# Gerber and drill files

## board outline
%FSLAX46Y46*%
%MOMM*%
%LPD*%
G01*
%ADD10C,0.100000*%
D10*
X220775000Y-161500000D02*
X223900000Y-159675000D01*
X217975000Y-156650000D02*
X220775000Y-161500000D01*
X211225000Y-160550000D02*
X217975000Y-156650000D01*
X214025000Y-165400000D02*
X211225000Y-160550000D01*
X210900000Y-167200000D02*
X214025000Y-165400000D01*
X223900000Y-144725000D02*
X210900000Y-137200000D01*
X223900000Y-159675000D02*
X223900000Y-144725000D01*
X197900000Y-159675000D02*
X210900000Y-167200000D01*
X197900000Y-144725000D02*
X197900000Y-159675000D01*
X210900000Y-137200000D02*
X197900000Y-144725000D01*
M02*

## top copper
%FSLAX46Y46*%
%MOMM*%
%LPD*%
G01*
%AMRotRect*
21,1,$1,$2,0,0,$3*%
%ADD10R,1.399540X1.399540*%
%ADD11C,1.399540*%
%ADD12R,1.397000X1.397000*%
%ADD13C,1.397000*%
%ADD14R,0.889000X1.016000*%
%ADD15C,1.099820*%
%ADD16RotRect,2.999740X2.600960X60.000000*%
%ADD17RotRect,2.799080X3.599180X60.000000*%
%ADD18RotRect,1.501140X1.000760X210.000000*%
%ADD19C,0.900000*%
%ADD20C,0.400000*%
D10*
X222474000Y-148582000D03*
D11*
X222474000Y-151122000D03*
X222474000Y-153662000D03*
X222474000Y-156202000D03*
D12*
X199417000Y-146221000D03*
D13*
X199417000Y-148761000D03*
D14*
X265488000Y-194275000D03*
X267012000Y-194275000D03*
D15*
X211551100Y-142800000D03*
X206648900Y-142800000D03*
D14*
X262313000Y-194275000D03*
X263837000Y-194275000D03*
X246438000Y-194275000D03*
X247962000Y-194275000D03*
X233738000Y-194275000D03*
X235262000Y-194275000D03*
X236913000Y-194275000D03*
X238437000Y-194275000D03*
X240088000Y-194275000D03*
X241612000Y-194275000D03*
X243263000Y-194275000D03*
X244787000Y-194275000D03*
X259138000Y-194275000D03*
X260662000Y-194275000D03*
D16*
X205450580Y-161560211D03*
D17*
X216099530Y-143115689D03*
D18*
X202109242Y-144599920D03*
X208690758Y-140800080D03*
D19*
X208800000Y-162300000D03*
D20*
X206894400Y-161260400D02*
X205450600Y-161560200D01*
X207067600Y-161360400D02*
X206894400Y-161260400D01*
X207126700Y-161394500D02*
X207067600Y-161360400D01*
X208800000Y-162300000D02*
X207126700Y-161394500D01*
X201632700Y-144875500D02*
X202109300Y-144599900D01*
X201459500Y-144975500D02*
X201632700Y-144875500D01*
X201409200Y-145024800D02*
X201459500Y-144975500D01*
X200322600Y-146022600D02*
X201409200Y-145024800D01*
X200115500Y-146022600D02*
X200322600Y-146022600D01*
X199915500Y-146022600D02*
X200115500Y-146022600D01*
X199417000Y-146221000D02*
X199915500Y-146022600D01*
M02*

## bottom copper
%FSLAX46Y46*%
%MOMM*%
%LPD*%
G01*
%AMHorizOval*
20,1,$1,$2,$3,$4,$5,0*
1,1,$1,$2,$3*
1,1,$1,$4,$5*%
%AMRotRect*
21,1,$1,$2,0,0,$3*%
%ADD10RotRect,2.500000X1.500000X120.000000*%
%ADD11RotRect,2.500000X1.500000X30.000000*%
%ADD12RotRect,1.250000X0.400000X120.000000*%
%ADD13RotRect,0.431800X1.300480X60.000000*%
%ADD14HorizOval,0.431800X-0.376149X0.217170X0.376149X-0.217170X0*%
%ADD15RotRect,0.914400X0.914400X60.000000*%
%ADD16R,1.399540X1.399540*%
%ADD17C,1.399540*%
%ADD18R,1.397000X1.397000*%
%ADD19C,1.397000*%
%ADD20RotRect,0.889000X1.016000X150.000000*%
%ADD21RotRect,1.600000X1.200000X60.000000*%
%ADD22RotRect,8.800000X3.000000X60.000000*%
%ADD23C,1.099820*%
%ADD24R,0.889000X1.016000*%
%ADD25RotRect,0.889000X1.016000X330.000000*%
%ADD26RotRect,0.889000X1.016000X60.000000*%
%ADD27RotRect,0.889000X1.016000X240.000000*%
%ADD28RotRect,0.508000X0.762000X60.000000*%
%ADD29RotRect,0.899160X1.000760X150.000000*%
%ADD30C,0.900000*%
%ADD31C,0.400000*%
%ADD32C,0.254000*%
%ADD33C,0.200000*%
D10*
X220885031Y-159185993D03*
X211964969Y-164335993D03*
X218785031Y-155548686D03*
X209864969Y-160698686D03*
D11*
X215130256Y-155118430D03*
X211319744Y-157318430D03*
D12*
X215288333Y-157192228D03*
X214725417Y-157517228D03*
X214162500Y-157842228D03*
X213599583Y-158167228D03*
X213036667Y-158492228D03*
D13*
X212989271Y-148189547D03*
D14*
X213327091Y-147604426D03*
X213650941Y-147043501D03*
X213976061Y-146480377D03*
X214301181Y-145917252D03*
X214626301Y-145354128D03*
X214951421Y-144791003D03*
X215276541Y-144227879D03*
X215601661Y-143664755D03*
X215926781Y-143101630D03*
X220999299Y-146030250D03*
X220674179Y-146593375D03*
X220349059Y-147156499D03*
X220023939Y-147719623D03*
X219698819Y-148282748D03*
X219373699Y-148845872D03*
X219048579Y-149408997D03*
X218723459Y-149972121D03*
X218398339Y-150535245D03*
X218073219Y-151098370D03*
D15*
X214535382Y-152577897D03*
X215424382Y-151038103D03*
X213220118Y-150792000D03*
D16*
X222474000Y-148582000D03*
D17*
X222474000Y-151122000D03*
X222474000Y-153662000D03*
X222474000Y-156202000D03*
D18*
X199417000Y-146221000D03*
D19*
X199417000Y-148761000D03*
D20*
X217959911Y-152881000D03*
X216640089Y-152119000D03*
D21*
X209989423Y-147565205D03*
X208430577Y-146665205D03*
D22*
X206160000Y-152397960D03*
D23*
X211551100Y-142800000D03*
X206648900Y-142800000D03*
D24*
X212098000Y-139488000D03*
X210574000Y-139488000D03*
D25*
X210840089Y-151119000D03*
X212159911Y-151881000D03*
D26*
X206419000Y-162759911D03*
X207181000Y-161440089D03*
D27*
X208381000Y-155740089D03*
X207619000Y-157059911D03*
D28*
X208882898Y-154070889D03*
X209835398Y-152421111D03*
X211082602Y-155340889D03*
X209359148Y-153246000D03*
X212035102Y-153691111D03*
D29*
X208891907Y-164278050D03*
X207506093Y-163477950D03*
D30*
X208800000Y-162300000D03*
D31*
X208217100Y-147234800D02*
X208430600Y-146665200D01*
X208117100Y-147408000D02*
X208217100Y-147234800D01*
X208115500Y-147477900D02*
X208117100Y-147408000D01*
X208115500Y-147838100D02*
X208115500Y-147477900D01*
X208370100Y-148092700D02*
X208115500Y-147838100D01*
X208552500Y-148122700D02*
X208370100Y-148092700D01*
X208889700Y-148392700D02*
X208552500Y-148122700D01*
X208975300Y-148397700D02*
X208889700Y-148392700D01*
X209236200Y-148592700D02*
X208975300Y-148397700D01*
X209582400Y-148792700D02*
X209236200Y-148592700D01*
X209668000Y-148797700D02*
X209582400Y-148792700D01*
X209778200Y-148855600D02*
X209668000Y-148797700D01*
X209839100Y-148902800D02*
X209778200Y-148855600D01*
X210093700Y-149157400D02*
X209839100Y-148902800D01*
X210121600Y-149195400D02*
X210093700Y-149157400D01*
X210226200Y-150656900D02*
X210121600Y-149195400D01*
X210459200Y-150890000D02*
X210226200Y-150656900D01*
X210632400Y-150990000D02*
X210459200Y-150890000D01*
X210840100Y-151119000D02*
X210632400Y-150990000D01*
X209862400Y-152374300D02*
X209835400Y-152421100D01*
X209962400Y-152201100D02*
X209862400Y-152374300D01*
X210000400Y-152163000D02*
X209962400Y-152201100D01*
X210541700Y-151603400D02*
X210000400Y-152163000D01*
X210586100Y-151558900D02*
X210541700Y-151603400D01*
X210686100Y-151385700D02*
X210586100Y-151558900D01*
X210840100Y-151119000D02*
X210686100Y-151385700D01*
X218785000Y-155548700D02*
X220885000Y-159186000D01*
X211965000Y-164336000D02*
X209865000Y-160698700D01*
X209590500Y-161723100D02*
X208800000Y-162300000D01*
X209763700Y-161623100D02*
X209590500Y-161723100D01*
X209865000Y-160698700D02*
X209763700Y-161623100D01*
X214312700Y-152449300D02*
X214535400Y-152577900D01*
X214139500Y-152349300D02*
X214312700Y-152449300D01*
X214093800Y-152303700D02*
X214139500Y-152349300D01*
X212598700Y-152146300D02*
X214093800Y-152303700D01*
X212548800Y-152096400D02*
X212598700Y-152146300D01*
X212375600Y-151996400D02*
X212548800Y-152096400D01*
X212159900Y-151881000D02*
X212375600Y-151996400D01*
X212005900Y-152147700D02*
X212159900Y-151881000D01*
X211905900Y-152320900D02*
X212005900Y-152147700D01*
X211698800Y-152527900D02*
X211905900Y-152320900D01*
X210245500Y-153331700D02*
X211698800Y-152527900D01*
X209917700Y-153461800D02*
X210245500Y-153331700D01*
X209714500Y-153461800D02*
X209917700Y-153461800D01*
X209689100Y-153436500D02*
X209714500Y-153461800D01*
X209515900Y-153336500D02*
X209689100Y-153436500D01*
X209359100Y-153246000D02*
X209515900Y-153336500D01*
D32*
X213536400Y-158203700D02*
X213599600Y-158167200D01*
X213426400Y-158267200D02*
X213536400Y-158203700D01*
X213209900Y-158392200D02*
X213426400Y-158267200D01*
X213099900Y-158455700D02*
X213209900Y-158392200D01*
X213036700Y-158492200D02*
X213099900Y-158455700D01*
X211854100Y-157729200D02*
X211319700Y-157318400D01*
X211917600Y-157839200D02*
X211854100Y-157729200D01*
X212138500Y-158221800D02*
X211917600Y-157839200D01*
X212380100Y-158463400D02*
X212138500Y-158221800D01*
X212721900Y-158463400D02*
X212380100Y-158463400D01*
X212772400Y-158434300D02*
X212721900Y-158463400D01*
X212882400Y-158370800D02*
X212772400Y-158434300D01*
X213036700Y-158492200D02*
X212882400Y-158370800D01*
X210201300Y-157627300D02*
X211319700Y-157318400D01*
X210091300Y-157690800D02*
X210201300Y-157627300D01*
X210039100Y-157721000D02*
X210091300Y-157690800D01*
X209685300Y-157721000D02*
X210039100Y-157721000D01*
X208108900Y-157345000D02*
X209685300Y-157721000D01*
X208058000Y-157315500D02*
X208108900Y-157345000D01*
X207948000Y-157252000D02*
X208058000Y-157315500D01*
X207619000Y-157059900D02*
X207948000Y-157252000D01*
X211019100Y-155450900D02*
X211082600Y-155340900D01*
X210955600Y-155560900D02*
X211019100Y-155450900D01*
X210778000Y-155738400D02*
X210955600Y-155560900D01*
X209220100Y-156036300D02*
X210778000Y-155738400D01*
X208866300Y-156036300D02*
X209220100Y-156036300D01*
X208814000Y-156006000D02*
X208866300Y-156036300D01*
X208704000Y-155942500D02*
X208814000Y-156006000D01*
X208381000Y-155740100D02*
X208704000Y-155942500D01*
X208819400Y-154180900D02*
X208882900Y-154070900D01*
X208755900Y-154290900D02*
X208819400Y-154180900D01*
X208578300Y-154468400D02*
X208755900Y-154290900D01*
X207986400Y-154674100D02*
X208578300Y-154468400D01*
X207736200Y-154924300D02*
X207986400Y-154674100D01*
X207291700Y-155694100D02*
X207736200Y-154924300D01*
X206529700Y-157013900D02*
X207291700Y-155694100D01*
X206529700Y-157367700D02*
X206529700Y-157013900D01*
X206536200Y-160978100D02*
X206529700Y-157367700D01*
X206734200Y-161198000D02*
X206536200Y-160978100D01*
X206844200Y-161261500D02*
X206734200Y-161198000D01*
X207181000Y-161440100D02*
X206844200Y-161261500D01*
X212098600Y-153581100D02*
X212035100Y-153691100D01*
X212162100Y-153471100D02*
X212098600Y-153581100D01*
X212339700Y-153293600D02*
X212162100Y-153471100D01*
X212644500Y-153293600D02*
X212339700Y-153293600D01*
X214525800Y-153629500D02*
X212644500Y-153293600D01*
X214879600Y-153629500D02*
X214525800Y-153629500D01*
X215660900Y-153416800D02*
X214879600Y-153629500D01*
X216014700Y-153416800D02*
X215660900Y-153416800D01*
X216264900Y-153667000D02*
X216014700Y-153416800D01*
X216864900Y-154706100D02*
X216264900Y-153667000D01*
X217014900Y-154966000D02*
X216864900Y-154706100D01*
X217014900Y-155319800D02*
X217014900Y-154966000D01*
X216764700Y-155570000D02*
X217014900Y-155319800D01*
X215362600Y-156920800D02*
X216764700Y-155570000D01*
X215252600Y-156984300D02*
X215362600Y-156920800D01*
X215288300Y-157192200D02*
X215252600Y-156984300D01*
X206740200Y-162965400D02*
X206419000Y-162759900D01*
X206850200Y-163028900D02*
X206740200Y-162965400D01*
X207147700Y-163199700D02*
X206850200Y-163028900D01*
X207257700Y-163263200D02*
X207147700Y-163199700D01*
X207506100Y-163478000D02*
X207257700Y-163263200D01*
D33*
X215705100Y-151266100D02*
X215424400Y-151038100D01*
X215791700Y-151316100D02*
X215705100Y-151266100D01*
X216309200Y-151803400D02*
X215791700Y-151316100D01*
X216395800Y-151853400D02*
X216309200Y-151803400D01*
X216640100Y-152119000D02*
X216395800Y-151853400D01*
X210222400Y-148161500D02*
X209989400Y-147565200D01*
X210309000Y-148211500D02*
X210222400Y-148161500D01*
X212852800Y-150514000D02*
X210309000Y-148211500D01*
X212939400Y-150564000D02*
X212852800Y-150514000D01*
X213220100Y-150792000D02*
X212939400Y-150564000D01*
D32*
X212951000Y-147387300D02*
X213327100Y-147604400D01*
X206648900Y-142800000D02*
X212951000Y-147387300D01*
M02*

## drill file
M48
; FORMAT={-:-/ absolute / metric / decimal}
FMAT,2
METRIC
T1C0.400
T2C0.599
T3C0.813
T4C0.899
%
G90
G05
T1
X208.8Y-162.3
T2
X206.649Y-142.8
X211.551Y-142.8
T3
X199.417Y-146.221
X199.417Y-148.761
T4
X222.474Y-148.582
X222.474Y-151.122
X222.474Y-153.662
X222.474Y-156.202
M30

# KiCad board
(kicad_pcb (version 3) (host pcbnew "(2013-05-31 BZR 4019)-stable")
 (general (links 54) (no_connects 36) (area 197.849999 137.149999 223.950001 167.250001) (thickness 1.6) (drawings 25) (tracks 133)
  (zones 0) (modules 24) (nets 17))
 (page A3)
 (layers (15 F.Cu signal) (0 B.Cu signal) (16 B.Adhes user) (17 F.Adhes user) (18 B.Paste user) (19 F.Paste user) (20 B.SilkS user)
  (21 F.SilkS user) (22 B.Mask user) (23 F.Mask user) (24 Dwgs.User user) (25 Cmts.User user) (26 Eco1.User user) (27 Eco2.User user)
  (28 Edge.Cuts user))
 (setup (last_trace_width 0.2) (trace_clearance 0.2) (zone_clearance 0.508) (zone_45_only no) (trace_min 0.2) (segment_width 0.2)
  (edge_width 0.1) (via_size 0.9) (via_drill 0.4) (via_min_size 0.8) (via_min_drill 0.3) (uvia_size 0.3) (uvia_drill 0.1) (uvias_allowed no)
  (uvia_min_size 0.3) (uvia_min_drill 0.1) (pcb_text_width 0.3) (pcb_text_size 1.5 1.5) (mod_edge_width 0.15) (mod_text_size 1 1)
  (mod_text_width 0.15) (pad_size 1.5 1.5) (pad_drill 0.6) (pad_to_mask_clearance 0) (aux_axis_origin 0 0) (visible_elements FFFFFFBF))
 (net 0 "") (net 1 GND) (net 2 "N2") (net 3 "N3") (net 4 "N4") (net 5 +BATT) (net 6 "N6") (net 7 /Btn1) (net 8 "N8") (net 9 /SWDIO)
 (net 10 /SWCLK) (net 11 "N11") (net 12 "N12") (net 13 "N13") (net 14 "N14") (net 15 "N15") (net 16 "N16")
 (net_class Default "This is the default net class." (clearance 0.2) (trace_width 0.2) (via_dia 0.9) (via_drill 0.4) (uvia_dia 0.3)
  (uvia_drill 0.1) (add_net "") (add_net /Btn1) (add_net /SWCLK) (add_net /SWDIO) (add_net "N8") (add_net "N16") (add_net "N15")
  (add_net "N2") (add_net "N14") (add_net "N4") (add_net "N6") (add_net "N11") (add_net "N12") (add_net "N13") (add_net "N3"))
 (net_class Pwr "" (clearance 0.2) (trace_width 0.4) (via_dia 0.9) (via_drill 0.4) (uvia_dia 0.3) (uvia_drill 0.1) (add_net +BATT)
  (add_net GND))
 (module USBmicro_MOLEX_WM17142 (layer B.Cu) (at 214.6 158.6 120)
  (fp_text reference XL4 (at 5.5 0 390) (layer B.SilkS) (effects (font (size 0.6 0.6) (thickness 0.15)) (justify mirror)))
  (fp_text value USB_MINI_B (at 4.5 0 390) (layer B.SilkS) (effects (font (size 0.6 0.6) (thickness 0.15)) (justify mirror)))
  (pad SHLD smd rect (at -3.65 5.15 120) (size 2.5 1.5) (layers B.Cu B.Paste B.Mask) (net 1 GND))
  (pad SHLD smd rect (at -3.65 -5.15 120) (size 2.5 1.5) (layers B.Cu B.Paste B.Mask) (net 1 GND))
  (pad SHLD smd rect (at 0.55 5.15 120) (size 2.5 1.5) (layers B.Cu B.Paste B.Mask) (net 1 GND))
  (pad SHLD smd rect (at 0.55 -5.15 120) (size 2.5 1.5) (layers B.Cu B.Paste B.Mask) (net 1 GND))
  (pad SHLD smd rect (at 2.75 2.2 30) (size 2.5 1.5) (layers B.Cu B.Paste B.Mask) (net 1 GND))
  (pad SHLD smd rect (at 2.75 -2.2 30) (size 2.5 1.5) (layers B.Cu B.Paste B.Mask) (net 1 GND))
  (pad 1 smd rect (at 0.875 1.3 120) (size 1.25 0.4) (layers B.Cu B.Paste B.Mask) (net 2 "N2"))
  (pad 2 smd rect (at 0.875 0.65 120) (size 1.25 0.4) (layers B.Cu B.Paste B.Mask))
  (pad 3 smd rect (at 0.875 0 120) (size 1.25 0.4) (layers B.Cu B.Paste B.Mask))
  (pad 4 smd rect (at 0.875 -0.65 120) (size 1.25 0.4) (layers B.Cu B.Paste B.Mask) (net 1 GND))
  (pad 5 smd rect (at 0.875 -1.3 120) (size 1.25 0.4) (layers B.Cu B.Paste B.Mask) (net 1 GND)))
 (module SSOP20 (layer B.Cu) (at 217 147.1 60)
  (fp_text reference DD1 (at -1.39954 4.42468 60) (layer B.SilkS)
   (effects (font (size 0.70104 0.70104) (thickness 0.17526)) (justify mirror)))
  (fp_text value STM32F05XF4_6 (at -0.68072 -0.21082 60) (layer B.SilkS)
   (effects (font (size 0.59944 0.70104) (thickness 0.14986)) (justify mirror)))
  (pad 1 smd rect (at -2.94894 -2.92862 60) (size 0.4318 1.30048) (layers B.Cu B.Paste B.Mask) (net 1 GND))
  (pad 2 smd oval (at -2.2733 -2.92862 60) (size 0.4318 1.30048) (layers B.Cu B.Paste B.Mask) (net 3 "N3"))
  (pad 3 smd oval (at -1.6256 -2.92862 60) (size 0.4318 1.30048) (layers B.Cu B.Paste B.Mask) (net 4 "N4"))
  (pad 4 smd oval (at -0.97536 -2.92862 60) (size 0.4318 1.30048) (layers B.Cu B.Paste B.Mask))
  (pad 5 smd oval (at -0.32512 -2.92862 60) (size 0.4318 1.30048) (layers B.Cu B.Paste B.Mask) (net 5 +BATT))
  (pad 6 smd oval (at 0.32512 -2.92862 60) (size 0.4318 1.30048) (layers B.Cu B.Paste B.Mask))
  (pad 7 smd oval (at 0.97536 -2.92862 60) (size 0.4318 1.30048) (layers B.Cu B.Paste B.Mask) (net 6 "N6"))
  (pad 8 smd oval (at 1.6256 -2.92862 60) (size 0.4318 1.30048) (layers B.Cu B.Paste B.Mask) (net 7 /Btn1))
  (pad 9 smd oval (at 2.27584 -2.92862 60) (size 0.4318 1.30048) (layers B.Cu B.Paste B.Mask))
  (pad 10 smd oval (at 2.92608 -2.92862 60) (size 0.4318 1.30048) (layers B.Cu B.Paste B.Mask))
  (pad 11 smd oval (at 2.92608 2.92862 60) (size 0.4318 1.30048) (layers B.Cu B.Paste B.Mask))
  (pad 12 smd oval (at 2.27584 2.92862 60) (size 0.4318 1.30048) (layers B.Cu B.Paste B.Mask))
  (pad 13 smd oval (at 1.6256 2.92862 60) (size 0.4318 1.30048) (layers B.Cu B.Paste B.Mask))
  (pad 14 smd oval (at 0.97536 2.92862 60) (size 0.4318 1.30048) (layers B.Cu B.Paste B.Mask))
  (pad 15 smd oval (at 0.32512 2.92862 60) (size 0.4318 1.30048) (layers B.Cu B.Paste B.Mask) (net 1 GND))
  (pad 16 smd oval (at -0.32512 2.92862 60) (size 0.4318 1.30048) (layers B.Cu B.Paste B.Mask) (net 5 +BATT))
  (pad 17 smd oval (at -0.97536 2.92862 60) (size 0.4318 1.30048) (layers B.Cu B.Paste B.Mask) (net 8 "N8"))
  (pad 18 smd oval (at -1.6256 2.92862 60) (size 0.4318 1.30048) (layers B.Cu B.Paste B.Mask))
  (pad 19 smd oval (at -2.27584 2.92862 60) (size 0.4318 1.30048) (layers B.Cu B.Paste B.Mask) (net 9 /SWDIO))
  (pad 20 smd oval (at -2.92608 2.92862 60) (size 0.4318 1.30048) (layers B.Cu B.Paste B.Mask) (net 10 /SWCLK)))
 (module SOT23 (layer B.Cu) (at 214.1 151.3 60)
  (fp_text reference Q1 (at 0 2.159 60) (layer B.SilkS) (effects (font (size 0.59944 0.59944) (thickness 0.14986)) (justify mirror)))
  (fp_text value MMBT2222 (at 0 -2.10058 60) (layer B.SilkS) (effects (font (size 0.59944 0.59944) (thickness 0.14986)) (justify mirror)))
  (pad 2 smd rect (at -0.889 1.016 60) (size 0.9144 0.9144) (layers B.Cu B.Paste B.Mask) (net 1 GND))
  (pad 1 smd rect (at 0.889 1.016 60) (size 0.9144 0.9144) (layers B.Cu B.Paste B.Mask) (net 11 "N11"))
  (pad 3 smd rect (at 0 -1.016 60) (size 0.9144 0.9144) (layers B.Cu B.Paste B.Mask) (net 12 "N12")))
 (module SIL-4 (layer F.Cu) (at 222.474 152.392 270)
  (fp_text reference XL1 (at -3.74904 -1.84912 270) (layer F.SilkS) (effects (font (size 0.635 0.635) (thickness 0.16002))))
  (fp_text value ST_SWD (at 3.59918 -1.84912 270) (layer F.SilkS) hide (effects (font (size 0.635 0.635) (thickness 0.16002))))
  (pad 1 thru_hole rect (at -3.81 0 270) (size 1.39954 1.39954) (drill 0.89916) (layers *.Cu *.Mask F.SilkS) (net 5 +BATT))
  (pad 2 thru_hole circle (at -1.27 0 270) (size 1.39954 1.39954) (drill 0.89916) (layers *.Cu *.Mask F.SilkS) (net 10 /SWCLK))
  (pad 3 thru_hole circle (at 1.27 0 270) (size 1.39954 1.39954) (drill 0.89916) (layers *.Cu *.Mask F.SilkS) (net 1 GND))
  (pad 4 thru_hole circle (at 3.81 0 270) (size 1.39954 1.39954) (drill 0.89916) (layers *.Cu *.Mask F.SilkS) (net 9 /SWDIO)))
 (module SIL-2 (layer F.Cu) (at 199.417 147.491 270)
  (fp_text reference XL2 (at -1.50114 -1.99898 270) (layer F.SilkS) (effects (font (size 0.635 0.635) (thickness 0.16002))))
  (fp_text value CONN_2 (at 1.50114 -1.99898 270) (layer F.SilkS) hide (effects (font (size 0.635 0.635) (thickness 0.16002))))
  (pad 1 thru_hole rect (at -1.27 0 270) (size 1.397 1.397) (drill 0.8128) (layers *.Cu *.Mask F.SilkS) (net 1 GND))
  (pad 2 thru_hole circle (at 1.27 0 270) (size 1.397 1.397) (drill 0.8128) (layers *.Cu *.Mask F.SilkS) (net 8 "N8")))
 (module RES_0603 (layer B.Cu) (at 217.3 152.5 150)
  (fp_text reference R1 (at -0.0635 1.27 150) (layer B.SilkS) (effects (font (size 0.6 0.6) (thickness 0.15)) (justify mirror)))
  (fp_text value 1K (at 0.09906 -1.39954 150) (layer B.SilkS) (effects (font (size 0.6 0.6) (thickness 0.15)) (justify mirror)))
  (pad 1 smd rect (at -0.762 0 150) (size 0.889 1.016) (layers B.Cu B.Paste B.Mask) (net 6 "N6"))
  (pad 2 smd rect (at 0.762 0 150) (size 0.889 1.016) (layers B.Cu B.Paste B.Mask) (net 11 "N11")))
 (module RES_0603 (layer F.Cu) (at 266.25 194.275)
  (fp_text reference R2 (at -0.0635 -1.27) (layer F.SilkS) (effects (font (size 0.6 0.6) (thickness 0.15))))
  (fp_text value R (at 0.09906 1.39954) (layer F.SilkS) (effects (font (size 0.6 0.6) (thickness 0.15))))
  (pad 1 smd rect (at -0.762 0) (size 0.889 1.016) (layers F.Cu F.Paste F.Mask) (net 4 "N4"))
  (pad 2 smd rect (at 0.762 0) (size 0.889 1.016) (layers F.Cu F.Paste F.Mask) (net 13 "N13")))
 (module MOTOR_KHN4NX (layer B.Cu) (at 209.31 146.942 60)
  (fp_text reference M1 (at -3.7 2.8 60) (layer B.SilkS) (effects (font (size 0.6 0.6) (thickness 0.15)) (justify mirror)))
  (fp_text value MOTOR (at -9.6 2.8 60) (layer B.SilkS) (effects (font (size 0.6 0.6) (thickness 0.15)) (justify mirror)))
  (pad 1 smd rect (at -0.2 0.9 60) (size 1.6 1.2) (layers B.Cu B.Paste B.Mask) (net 12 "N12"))
  (pad 2 smd rect (at -0.2 -0.9 60) (size 1.6 1.2) (layers B.Cu B.Paste B.Mask) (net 5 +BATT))
  (pad PAD smd rect (at -6.3 0 60) (size 8.8 3) (layers B.Cu B.Paste B.Mask)))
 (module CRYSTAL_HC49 (layer B.Cu) (at 209.1 142.8 180)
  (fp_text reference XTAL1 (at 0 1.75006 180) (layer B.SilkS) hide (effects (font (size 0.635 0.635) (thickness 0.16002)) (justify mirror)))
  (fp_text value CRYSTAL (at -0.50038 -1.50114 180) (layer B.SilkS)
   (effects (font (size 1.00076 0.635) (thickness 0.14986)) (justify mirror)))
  (pad 1 thru_hole circle (at -2.4511 0 90) (size 1.09982 1.09982) (drill 0.59944) (layers *.Cu *.Mask B.SilkS) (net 13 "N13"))
  (pad 2 thru_hole circle (at 2.4511 0 90) (size 1.09982 1.09982) (drill 0.59944) (layers *.Cu *.Mask B.SilkS) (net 3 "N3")))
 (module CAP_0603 (layer F.Cu) (at 263.075 194.275)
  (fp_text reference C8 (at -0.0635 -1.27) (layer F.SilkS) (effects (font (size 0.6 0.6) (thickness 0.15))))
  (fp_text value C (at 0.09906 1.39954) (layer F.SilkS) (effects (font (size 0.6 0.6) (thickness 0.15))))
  (pad 1 smd rect (at -0.762 0) (size 0.889 1.016) (layers F.Cu F.Paste F.Mask) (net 3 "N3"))
  (pad 2 smd rect (at 0.762 0) (size 0.889 1.016) (layers F.Cu F.Paste F.Mask) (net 1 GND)))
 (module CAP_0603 (layer B.Cu) (at 211.336 139.488 180)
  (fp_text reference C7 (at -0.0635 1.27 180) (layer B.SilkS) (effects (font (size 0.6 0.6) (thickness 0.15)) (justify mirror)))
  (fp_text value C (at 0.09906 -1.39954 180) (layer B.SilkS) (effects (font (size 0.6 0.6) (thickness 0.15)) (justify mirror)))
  (pad 1 smd rect (at -0.762 0 180) (size 0.889 1.016) (layers B.Cu B.Paste B.Mask) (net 13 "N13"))
  (pad 2 smd rect (at 0.762 0 180) (size 0.889 1.016) (layers B.Cu B.Paste B.Mask) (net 1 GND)))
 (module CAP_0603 (layer F.Cu) (at 247.2 194.275)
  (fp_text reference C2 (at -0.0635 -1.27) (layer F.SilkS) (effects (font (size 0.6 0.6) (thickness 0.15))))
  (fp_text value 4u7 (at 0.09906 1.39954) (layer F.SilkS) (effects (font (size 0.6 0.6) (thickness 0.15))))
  (pad 1 smd rect (at -0.762 0) (size 0.889 1.016) (layers F.Cu F.Paste F.Mask) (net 5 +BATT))
  (pad 2 smd rect (at 0.762 0) (size 0.889 1.016) (layers F.Cu F.Paste F.Mask) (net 1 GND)))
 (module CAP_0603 (layer B.Cu) (at 211.5 151.5 330)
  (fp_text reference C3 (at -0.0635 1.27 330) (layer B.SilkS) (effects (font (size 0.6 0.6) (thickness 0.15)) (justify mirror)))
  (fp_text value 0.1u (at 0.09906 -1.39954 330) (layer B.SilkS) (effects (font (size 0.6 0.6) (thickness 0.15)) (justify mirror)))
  (pad 1 smd rect (at -0.762 0 330) (size 0.889 1.016) (layers B.Cu B.Paste B.Mask) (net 5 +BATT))
  (pad 2 smd rect (at 0.762 0 330) (size 0.889 1.016) (layers B.Cu B.Paste B.Mask) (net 1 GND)))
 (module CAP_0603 (layer F.Cu) (at 234.5 194.275)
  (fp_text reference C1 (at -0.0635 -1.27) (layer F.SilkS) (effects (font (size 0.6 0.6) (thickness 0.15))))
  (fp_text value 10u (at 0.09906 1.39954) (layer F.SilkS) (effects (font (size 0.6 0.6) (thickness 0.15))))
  (pad 1 smd rect (at -0.762 0) (size 0.889 1.016) (layers F.Cu F.Paste F.Mask) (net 5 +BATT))
  (pad 2 smd rect (at 0.762 0) (size 0.889 1.016) (layers F.Cu F.Paste F.Mask) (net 1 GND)))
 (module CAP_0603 (layer F.Cu) (at 237.675 194.275)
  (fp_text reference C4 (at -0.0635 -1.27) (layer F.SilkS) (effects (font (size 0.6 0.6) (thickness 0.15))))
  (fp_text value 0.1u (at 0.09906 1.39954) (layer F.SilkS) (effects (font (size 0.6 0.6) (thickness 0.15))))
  (pad 1 smd rect (at -0.762 0) (size 0.889 1.016) (layers F.Cu F.Paste F.Mask) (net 5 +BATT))
  (pad 2 smd rect (at 0.762 0) (size 0.889 1.016) (layers F.Cu F.Paste F.Mask) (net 1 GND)))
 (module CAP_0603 (layer F.Cu) (at 240.85 194.275)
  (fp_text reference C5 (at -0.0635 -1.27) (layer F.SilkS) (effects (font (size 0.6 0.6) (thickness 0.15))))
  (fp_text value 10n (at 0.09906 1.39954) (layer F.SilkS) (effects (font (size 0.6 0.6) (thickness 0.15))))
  (pad 1 smd rect (at -0.762 0) (size 0.889 1.016) (layers F.Cu F.Paste F.Mask) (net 5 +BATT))
  (pad 2 smd rect (at 0.762 0) (size 0.889 1.016) (layers F.Cu F.Paste F.Mask) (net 1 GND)))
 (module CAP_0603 (layer F.Cu) (at 244.025 194.275)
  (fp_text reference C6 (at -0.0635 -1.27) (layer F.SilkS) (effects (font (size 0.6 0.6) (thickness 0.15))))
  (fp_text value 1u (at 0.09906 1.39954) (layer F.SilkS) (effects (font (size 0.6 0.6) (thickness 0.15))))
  (pad 1 smd rect (at -0.762 0) (size 0.889 1.016) (layers F.Cu F.Paste F.Mask) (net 5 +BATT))
  (pad 2 smd rect (at 0.762 0) (size 0.889 1.016) (layers F.Cu F.Paste F.Mask) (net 1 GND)))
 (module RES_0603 (layer B.Cu) (at 206.8 162.1 60)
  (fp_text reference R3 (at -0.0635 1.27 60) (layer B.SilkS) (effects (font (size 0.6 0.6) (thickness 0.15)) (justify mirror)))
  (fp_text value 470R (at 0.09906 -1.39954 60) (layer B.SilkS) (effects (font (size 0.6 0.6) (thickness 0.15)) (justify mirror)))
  (pad 1 smd rect (at -0.762 0 60) (size 0.889 1.016) (layers B.Cu B.Paste B.Mask) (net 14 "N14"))
  (pad 2 smd rect (at 0.762 0 60) (size 0.889 1.016) (layers B.Cu B.Paste B.Mask) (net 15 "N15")))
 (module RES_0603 (layer B.Cu) (at 208 156.4 240)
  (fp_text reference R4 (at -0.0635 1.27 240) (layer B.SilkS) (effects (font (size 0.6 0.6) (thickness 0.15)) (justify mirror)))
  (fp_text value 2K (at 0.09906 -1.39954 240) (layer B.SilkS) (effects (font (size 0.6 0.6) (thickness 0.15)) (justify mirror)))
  (pad 1 smd rect (at -0.762 0 240) (size 0.889 1.016) (layers B.Cu B.Paste B.Mask) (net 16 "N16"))
  (pad 2 smd rect (at 0.762 0 240) (size 0.889 1.016) (layers B.Cu B.Paste B.Mask) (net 1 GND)))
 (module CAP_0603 (layer F.Cu) (at 259.9 194.275)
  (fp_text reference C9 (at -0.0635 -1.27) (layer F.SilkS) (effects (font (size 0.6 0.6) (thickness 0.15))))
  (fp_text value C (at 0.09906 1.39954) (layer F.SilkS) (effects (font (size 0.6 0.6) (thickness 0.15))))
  (pad 1 smd rect (at -0.762 0) (size 0.889 1.016) (layers F.Cu F.Paste F.Mask) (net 5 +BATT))
  (pad 2 smd rect (at 0.762 0) (size 0.889 1.016) (layers F.Cu F.Paste F.Mask) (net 1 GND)))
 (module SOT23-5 (layer B.Cu) (at 210.459 153.881 60)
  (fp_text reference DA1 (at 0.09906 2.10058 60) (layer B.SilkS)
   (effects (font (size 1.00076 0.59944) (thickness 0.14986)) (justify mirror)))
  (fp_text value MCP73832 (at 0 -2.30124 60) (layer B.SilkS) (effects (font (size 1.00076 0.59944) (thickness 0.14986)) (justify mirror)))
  (pad 1 smd rect (at -0.9525 -1.27 60) (size 0.508 0.762) (layers B.Cu B.Paste B.Mask) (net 15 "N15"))
  (pad 3 smd rect (at 0.9525 -1.27 60) (size 0.508 0.762) (layers B.Cu B.Paste B.Mask) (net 5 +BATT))
  (pad 5 smd rect (at -0.9525 1.27 60) (size 0.508 0.762) (layers B.Cu B.Paste B.Mask) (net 16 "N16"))
  (pad 2 smd rect (at 0 -1.27 60) (size 0.508 0.762) (layers B.Cu B.Paste B.Mask) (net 1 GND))
  (pad 4 smd rect (at 0.9525 1.27 60) (size 0.508 0.762) (layers B.Cu B.Paste B.Mask) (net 2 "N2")))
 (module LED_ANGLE (layer B.Cu) (at 208.199 163.878 150)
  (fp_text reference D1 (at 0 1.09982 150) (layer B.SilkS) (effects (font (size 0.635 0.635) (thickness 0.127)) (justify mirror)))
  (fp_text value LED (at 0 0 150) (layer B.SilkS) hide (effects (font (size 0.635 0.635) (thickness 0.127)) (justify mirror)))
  (pad A smd rect (at -0.8001 0 150) (size 0.89916 1.00076) (layers B.Cu B.Paste B.Mask) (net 2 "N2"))
  (pad C smd rect (at 0.8001 0 150) (size 0.89916 1.00076) (layers B.Cu B.Paste B.Mask) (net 14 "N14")))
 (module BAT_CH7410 (layer F.Cu) (at 209.7 154.2 60)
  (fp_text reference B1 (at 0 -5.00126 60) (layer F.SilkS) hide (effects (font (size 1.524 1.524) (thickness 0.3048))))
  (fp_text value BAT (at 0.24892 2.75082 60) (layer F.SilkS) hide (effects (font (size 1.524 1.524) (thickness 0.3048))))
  (pad C smd rect (at -8.49884 0 60) (size 2.99974 2.60096) (layers F.Cu F.Paste F.Mask) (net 1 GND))
  (pad A smd rect (at 12.79906 0 60) (size 2.79908 3.59918) (layers F.Cu F.Paste F.Mask) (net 5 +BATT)))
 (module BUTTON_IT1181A (layer F.Cu) (at 205.4 142.7 210)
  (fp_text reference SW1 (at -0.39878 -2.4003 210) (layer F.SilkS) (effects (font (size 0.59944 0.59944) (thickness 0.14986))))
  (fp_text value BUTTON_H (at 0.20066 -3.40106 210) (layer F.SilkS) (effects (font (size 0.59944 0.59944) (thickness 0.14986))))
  (pad 2 smd rect (at 3.79984 0 210) (size 1.50114 1.00076) (layers F.Cu F.Paste F.Mask) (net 1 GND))
  (pad 1 smd rect (at -3.79984 0 210) (size 1.50114 1.00076) (layers F.Cu F.Paste F.Mask) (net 7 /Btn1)))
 (gr_line (start 220.775 161.5) (end 223.9 159.675) (angle 90) (layer Edge.Cuts) (width 0.1))
 (gr_line (start 217.975 156.65) (end 220.775 161.5) (angle 90) (layer Edge.Cuts) (width 0.1))
 (gr_line (start 211.225 160.55) (end 217.975 156.65) (angle 90) (layer Edge.Cuts) (width 0.1))
 (gr_line (start 214.025 165.4) (end 211.225 160.55) (angle 90) (layer Edge.Cuts) (width 0.1))
 (gr_line (start 210.9 167.2) (end 214.025 165.4) (angle 90) (layer Edge.Cuts) (width 0.1))
 (gr_line (start 223.9 144.725) (end 210.9 137.2) (angle 90) (layer Edge.Cuts) (width 0.1))
 (gr_line (start 223.9 159.675) (end 223.9 144.725) (angle 90) (layer Edge.Cuts) (width 0.1))
 (gr_line (start 197.9 159.675) (end 210.9 167.2) (angle 90) (layer Edge.Cuts) (width 0.1))
 (gr_line (start 197.9 144.725) (end 197.9 159.675) (angle 90) (layer Edge.Cuts) (width 0.1))
 (gr_line (start 210.9 137.2) (end 197.9 144.725) (angle 90) (layer Edge.Cuts) (width 0.1))
 (segment (start 208.2171 147.2348) (end 208.4306 146.6652) (width 0.4) (layer B.Cu) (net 5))
 (segment (start 208.1171 147.408) (end 208.2171 147.2348) (width 0.4) (layer B.Cu) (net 5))
 (segment (start 208.1155 147.4779) (end 208.1171 147.408) (width 0.4) (layer B.Cu) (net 5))
 (segment (start 208.1155 147.8381) (end 208.1155 147.4779) (width 0.4) (layer B.Cu) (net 5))
 (segment (start 208.3701 148.0927) (end 208.1155 147.8381) (width 0.4) (layer B.Cu) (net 5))
 (segment (start 208.5525 148.1227) (end 208.3701 148.0927) (width 0.4) (layer B.Cu) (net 5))
 (segment (start 208.8897 148.3927) (end 208.5525 148.1227) (width 0.4) (layer B.Cu) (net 5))
 (segment (start 208.9753 148.3977) (end 208.8897 148.3927) (width 0.4) (layer B.Cu) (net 5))
 (segment (start 209.2362 148.5927) (end 208.9753 148.3977) (width 0.4) (layer B.Cu) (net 5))
 (segment (start 209.5824 148.7927) (end 209.2362 148.5927) (width 0.4) (layer B.Cu) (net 5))
 (segment (start 209.668 148.7977) (end 209.5824 148.7927) (width 0.4) (layer B.Cu) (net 5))
 (segment (start 209.7782 148.8556) (end 209.668 148.7977) (width 0.4) (layer B.Cu) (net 5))
 (segment (start 209.8391 148.9028) (end 209.7782 148.8556) (width 0.4) (layer B.Cu) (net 5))
 (segment (start 210.0937 149.1574) (end 209.8391 148.9028) (width 0.4) (layer B.Cu) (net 5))
 (segment (start 210.1216 149.1954) (end 210.0937 149.1574) (width 0.4) (layer B.Cu) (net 5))
 (segment (start 210.2262 150.6569) (end 210.1216 149.1954) (width 0.4) (layer B.Cu) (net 5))
 (segment (start 210.4592 150.89) (end 210.2262 150.6569) (width 0.4) (layer B.Cu) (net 5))
 (segment (start 210.6324 150.99) (end 210.4592 150.89) (width 0.4) (layer B.Cu) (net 5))
 (segment (start 210.8401 151.119) (end 210.6324 150.99) (width 0.4) (layer B.Cu) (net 5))
 (segment (start 209.8624 152.3743) (end 209.8354 152.4211) (width 0.4) (layer B.Cu) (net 5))
 (segment (start 209.9624 152.2011) (end 209.8624 152.3743) (width 0.4) (layer B.Cu) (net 5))
 (segment (start 210.0004 152.163) (end 209.9624 152.2011) (width 0.4) (layer B.Cu) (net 5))
 (segment (start 210.5417 151.6034) (end 210.0004 152.163) (width 0.4) (layer B.Cu) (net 5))
 (segment (start 210.5861 151.5589) (end 210.5417 151.6034) (width 0.4) (layer B.Cu) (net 5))
 (segment (start 210.6861 151.3857) (end 210.5861 151.5589) (width 0.4) (layer B.Cu) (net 5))
 (segment (start 210.8401 151.119) (end 210.6861 151.3857) (width 0.4) (layer B.Cu) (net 5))
 (segment (start 218.785 155.5487) (end 220.885 159.186) (width 0.4) (layer B.Cu) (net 1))
 (via (at 208.8 162.3) (size 0.9) (layers F.Cu B.Cu) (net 1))
 (segment (start 211.965 164.336) (end 209.865 160.6987) (width 0.4) (layer B.Cu) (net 1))
 (segment (start 209.5905 161.7231) (end 208.8 162.3) (width 0.4) (layer B.Cu) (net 1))
 (segment (start 209.7637 161.6231) (end 209.5905 161.7231) (width 0.4) (layer B.Cu) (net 1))
 (segment (start 209.865 160.6987) (end 209.7637 161.6231) (width 0.4) (layer B.Cu) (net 1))
 (segment (start 214.3127 152.4493) (end 214.5354 152.5779) (width 0.4) (layer B.Cu) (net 1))
 (segment (start 214.1395 152.3493) (end 214.3127 152.4493) (width 0.4) (layer B.Cu) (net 1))
 (segment (start 214.0938 152.3037) (end 214.1395 152.3493) (width 0.4) (layer B.Cu) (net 1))
 (segment (start 212.5987 152.1463) (end 214.0938 152.3037) (width 0.4) (layer B.Cu) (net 1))
 (segment (start 212.5488 152.0964) (end 212.5987 152.1463) (width 0.4) (layer B.Cu) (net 1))
 (segment (start 212.3756 151.9964) (end 212.5488 152.0964) (width 0.4) (layer B.Cu) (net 1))
 (segment (start 212.1599 151.881) (end 212.3756 151.9964) (width 0.4) (layer B.Cu) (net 1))
 (segment (start 212.0059 152.1477) (end 212.1599 151.881) (width 0.4) (layer B.Cu) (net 1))
 (segment (start 211.9059 152.3209) (end 212.0059 152.1477) (width 0.4) (layer B.Cu) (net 1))
 (segment (start 211.6988 152.5279) (end 211.9059 152.3209) (width 0.4) (layer B.Cu) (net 1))
 (segment (start 210.2455 153.3317) (end 211.6988 152.5279) (width 0.4) (layer B.Cu) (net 1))
 (segment (start 209.9177 153.4618) (end 210.2455 153.3317) (width 0.4) (layer B.Cu) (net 1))
 (segment (start 209.7145 153.4618) (end 209.9177 153.4618) (width 0.4) (layer B.Cu) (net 1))
 (segment (start 209.6891 153.4365) (end 209.7145 153.4618) (width 0.4) (layer B.Cu) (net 1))
 (segment (start 209.5159 153.3365) (end 209.6891 153.4365) (width 0.4) (layer B.Cu) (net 1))
 (segment (start 209.3591 153.246) (end 209.5159 153.3365) (width 0.4) (layer B.Cu) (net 1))
 (segment (start 213.5364 158.2037) (end 213.5996 158.1672) (width 0.254) (layer B.Cu) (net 1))
 (segment (start 213.4264 158.2672) (end 213.5364 158.2037) (width 0.254) (layer B.Cu) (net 1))
 (segment (start 213.2099 158.3922) (end 213.4264 158.2672) (width 0.254) (layer B.Cu) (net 1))
 (segment (start 213.0999 158.4557) (end 213.2099 158.3922) (width 0.254) (layer B.Cu) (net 1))
 (segment (start 213.0367 158.4922) (end 213.0999 158.4557) (width 0.254) (layer B.Cu) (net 1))
 (segment (start 211.8541 157.7292) (end 211.3197 157.3184) (width 0.254) (layer B.Cu) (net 1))
 (segment (start 211.9176 157.8392) (end 211.8541 157.7292) (width 0.254) (layer B.Cu) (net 1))
 (segment (start 212.1385 158.2218) (end 211.9176 157.8392) (width 0.254) (layer B.Cu) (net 1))
 (segment (start 212.3801 158.4634) (end 212.1385 158.2218) (width 0.254) (layer B.Cu) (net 1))
 (segment (start 212.7219 158.4634) (end 212.3801 158.4634) (width 0.254) (layer B.Cu) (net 1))
 (segment (start 212.7724 158.4343) (end 212.7219 158.4634) (width 0.254) (layer B.Cu) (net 1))
 (segment (start 212.8824 158.3708) (end 212.7724 158.4343) (width 0.254) (layer B.Cu) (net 1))
 (segment (start 213.0367 158.4922) (end 212.8824 158.3708) (width 0.254) (layer B.Cu) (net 1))
 (segment (start 210.2013 157.6273) (end 211.3197 157.3184) (width 0.254) (layer B.Cu) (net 1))
 (segment (start 210.0913 157.6908) (end 210.2013 157.6273) (width 0.254) (layer B.Cu) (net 1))
 (segment (start 210.0391 157.721) (end 210.0913 157.6908) (width 0.254) (layer B.Cu) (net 1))
 (segment (start 209.6853 157.721) (end 210.0391 157.721) (width 0.254) (layer B.Cu) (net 1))
 (segment (start 208.1089 157.345) (end 209.6853 157.721) (width 0.254) (layer B.Cu) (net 1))
 (segment (start 208.058 157.3155) (end 208.1089 157.345) (width 0.254) (layer B.Cu) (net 1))
 (segment (start 207.948 157.252) (end 208.058 157.3155) (width 0.254) (layer B.Cu) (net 1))
 (segment (start 207.619 157.0599) (end 207.948 157.252) (width 0.254) (layer B.Cu) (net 1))
 (segment (start 206.8944 161.2604) (end 205.4506 161.5602) (width 0.4) (layer F.Cu) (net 1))
 (segment (start 207.0676 161.3604) (end 206.8944 161.2604) (width 0.4) (layer F.Cu) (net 1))
 (segment (start 207.1267 161.3945) (end 207.0676 161.3604) (width 0.4) (layer F.Cu) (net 1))
 (segment (start 208.8 162.3) (end 207.1267 161.3945) (width 0.4) (layer F.Cu) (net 1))
 (segment (start 201.6327 144.8755) (end 202.1093 144.5999) (width 0.4) (layer F.Cu) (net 1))
 (segment (start 201.4595 144.9755) (end 201.6327 144.8755) (width 0.4) (layer F.Cu) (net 1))
 (segment (start 201.4092 145.0248) (end 201.4595 144.9755) (width 0.4) (layer F.Cu) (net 1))
 (segment (start 200.3226 146.0226) (end 201.4092 145.0248) (width 0.4) (layer F.Cu) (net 1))
 (segment (start 200.1155 146.0226) (end 200.3226 146.0226) (width 0.4) (layer F.Cu) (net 1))
 (segment (start 199.9155 146.0226) (end 200.1155 146.0226) (width 0.4) (layer F.Cu) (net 1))
 (segment (start 199.417 146.221) (end 199.9155 146.0226) (width 0.4) (layer F.Cu) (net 1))
 (segment (start 211.0191 155.4509) (end 211.0826 155.3409) (width 0.254) (layer B.Cu) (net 16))
 (segment (start 210.9556 155.5609) (end 211.0191 155.4509) (width 0.254) (layer B.Cu) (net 16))
 (segment (start 210.778 155.7384) (end 210.9556 155.5609) (width 0.254) (layer B.Cu) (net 16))
 (segment (start 209.2201 156.0363) (end 210.778 155.7384) (width 0.254) (layer B.Cu) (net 16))
 (segment (start 208.8663 156.0363) (end 209.2201 156.0363) (width 0.254) (layer B.Cu) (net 16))
 (segment (start 208.814 156.006) (end 208.8663 156.0363) (width 0.254) (layer B.Cu) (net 16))
 (segment (start 208.704 155.9425) (end 208.814 156.006) (width 0.254) (layer B.Cu) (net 16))
 (segment (start 208.381 155.7401) (end 208.704 155.9425) (width 0.254) (layer B.Cu) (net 16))
 (segment (start 208.8194 154.1809) (end 208.8829 154.0709) (width 0.254) (layer B.Cu) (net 15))
 (segment (start 208.7559 154.2909) (end 208.8194 154.1809) (width 0.254) (layer B.Cu) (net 15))
 (segment (start 208.5783 154.4684) (end 208.7559 154.2909) (width 0.254) (layer B.Cu) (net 15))
 (segment (start 207.9864 154.6741) (end 208.5783 154.4684) (width 0.254) (layer B.Cu) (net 15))
 (segment (start 207.7362 154.9243) (end 207.9864 154.6741) (width 0.254) (layer B.Cu) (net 15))
 (segment (start 207.2917 155.6941) (end 207.7362 154.9243) (width 0.254) (layer B.Cu) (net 15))
 (segment (start 206.5297 157.0139) (end 207.2917 155.6941) (width 0.254) (layer B.Cu) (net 15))
 (segment (start 206.5297 157.3677) (end 206.5297 157.0139) (width 0.254) (layer B.Cu) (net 15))
 (segment (start 206.5362 160.9781) (end 206.5297 157.3677) (width 0.254) (layer B.Cu) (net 15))
 (segment (start 206.7342 161.198) (end 206.5362 160.9781) (width 0.254) (layer B.Cu) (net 15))
 (segment (start 206.8442 161.2615) (end 206.7342 161.198) (width 0.254) (layer B.Cu) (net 15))
 (segment (start 207.181 161.4401) (end 206.8442 161.2615) (width 0.254) (layer B.Cu) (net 15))
 (segment (start 212.0986 153.5811) (end 212.0351 153.6911) (width 0.254) (layer B.Cu) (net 2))
 (segment (start 212.1621 153.4711) (end 212.0986 153.5811) (width 0.254) (layer B.Cu) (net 2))
 (segment (start 212.3397 153.2936) (end 212.1621 153.4711) (width 0.254) (layer B.Cu) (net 2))
 (segment (start 212.6445 153.2936) (end 212.3397 153.2936) (width 0.254) (layer B.Cu) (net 2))
 (segment (start 214.5258 153.6295) (end 212.6445 153.2936) (width 0.254) (layer B.Cu) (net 2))
 (segment (start 214.8796 153.6295) (end 214.5258 153.6295) (width 0.254) (layer B.Cu) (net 2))
 (segment (start 215.6609 153.4168) (end 214.8796 153.6295) (width 0.254) (layer B.Cu) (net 2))
 (segment (start 216.0147 153.4168) (end 215.6609 153.4168) (width 0.254) (layer B.Cu) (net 2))
 (segment (start 216.2649 153.667) (end 216.0147 153.4168) (width 0.254) (layer B.Cu) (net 2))
 (segment (start 216.8649 154.7061) (end 216.2649 153.667) (width 0.254) (layer B.Cu) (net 2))
 (segment (start 217.0149 154.966) (end 216.8649 154.7061) (width 0.254) (layer B.Cu) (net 2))
 (segment (start 217.0149 155.3198) (end 217.0149 154.966) (width 0.254) (layer B.Cu) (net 2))
 (segment (start 216.7647 155.57) (end 217.0149 155.3198) (width 0.254) (layer B.Cu) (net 2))
 (segment (start 215.3626 156.9208) (end 216.7647 155.57) (width 0.254) (layer B.Cu) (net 2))
 (segment (start 215.2526 156.9843) (end 215.3626 156.9208) (width 0.254) (layer B.Cu) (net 2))
 (segment (start 215.2883 157.1922) (end 215.2526 156.9843) (width 0.254) (layer B.Cu) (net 2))
 (segment (start 206.7402 162.9654) (end 206.419 162.7599) (width 0.254) (layer B.Cu) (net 14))
 (segment (start 206.8502 163.0289) (end 206.7402 162.9654) (width 0.254) (layer B.Cu) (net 14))
 (segment (start 207.1477 163.1997) (end 206.8502 163.0289) (width 0.254) (layer B.Cu) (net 14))
 (segment (start 207.2577 163.2632) (end 207.1477 163.1997) (width 0.254) (layer B.Cu) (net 14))
 (segment (start 207.5061 163.478) (end 207.2577 163.2632) (width 0.254) (layer B.Cu) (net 14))
 (segment (start 215.7051 151.2661) (end 215.4244 151.0381) (width 0.2) (layer B.Cu) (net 11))
 (segment (start 215.7917 151.3161) (end 215.7051 151.2661) (width 0.2) (layer B.Cu) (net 11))
 (segment (start 216.3092 151.8034) (end 215.7917 151.3161) (width 0.2) (layer B.Cu) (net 11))
 (segment (start 216.3958 151.8534) (end 216.3092 151.8034) (width 0.2) (layer B.Cu) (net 11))
 (segment (start 216.6401 152.119) (end 216.3958 151.8534) (width 0.2) (layer B.Cu) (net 11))
 (segment (start 210.2224 148.1615) (end 209.9894 147.5652) (width 0.2) (layer B.Cu) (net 12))
 (segment (start 210.309 148.2115) (end 210.2224 148.1615) (width 0.2) (layer B.Cu) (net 12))
 (segment (start 212.8528 150.514) (end 210.309 148.2115) (width 0.2) (layer B.Cu) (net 12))
 (segment (start 212.9394 150.564) (end 212.8528 150.514) (width 0.2) (layer B.Cu) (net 12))
 (segment (start 213.2201 150.792) (end 212.9394 150.564) (width 0.2) (layer B.Cu) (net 12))
 (segment (start 212.951 147.3873) (end 213.3271 147.6044) (width 0.254) (layer B.Cu) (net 3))
 (segment (start 206.6489 142.8) (end 212.951 147.3873) (width 0.254) (layer B.Cu) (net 3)))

